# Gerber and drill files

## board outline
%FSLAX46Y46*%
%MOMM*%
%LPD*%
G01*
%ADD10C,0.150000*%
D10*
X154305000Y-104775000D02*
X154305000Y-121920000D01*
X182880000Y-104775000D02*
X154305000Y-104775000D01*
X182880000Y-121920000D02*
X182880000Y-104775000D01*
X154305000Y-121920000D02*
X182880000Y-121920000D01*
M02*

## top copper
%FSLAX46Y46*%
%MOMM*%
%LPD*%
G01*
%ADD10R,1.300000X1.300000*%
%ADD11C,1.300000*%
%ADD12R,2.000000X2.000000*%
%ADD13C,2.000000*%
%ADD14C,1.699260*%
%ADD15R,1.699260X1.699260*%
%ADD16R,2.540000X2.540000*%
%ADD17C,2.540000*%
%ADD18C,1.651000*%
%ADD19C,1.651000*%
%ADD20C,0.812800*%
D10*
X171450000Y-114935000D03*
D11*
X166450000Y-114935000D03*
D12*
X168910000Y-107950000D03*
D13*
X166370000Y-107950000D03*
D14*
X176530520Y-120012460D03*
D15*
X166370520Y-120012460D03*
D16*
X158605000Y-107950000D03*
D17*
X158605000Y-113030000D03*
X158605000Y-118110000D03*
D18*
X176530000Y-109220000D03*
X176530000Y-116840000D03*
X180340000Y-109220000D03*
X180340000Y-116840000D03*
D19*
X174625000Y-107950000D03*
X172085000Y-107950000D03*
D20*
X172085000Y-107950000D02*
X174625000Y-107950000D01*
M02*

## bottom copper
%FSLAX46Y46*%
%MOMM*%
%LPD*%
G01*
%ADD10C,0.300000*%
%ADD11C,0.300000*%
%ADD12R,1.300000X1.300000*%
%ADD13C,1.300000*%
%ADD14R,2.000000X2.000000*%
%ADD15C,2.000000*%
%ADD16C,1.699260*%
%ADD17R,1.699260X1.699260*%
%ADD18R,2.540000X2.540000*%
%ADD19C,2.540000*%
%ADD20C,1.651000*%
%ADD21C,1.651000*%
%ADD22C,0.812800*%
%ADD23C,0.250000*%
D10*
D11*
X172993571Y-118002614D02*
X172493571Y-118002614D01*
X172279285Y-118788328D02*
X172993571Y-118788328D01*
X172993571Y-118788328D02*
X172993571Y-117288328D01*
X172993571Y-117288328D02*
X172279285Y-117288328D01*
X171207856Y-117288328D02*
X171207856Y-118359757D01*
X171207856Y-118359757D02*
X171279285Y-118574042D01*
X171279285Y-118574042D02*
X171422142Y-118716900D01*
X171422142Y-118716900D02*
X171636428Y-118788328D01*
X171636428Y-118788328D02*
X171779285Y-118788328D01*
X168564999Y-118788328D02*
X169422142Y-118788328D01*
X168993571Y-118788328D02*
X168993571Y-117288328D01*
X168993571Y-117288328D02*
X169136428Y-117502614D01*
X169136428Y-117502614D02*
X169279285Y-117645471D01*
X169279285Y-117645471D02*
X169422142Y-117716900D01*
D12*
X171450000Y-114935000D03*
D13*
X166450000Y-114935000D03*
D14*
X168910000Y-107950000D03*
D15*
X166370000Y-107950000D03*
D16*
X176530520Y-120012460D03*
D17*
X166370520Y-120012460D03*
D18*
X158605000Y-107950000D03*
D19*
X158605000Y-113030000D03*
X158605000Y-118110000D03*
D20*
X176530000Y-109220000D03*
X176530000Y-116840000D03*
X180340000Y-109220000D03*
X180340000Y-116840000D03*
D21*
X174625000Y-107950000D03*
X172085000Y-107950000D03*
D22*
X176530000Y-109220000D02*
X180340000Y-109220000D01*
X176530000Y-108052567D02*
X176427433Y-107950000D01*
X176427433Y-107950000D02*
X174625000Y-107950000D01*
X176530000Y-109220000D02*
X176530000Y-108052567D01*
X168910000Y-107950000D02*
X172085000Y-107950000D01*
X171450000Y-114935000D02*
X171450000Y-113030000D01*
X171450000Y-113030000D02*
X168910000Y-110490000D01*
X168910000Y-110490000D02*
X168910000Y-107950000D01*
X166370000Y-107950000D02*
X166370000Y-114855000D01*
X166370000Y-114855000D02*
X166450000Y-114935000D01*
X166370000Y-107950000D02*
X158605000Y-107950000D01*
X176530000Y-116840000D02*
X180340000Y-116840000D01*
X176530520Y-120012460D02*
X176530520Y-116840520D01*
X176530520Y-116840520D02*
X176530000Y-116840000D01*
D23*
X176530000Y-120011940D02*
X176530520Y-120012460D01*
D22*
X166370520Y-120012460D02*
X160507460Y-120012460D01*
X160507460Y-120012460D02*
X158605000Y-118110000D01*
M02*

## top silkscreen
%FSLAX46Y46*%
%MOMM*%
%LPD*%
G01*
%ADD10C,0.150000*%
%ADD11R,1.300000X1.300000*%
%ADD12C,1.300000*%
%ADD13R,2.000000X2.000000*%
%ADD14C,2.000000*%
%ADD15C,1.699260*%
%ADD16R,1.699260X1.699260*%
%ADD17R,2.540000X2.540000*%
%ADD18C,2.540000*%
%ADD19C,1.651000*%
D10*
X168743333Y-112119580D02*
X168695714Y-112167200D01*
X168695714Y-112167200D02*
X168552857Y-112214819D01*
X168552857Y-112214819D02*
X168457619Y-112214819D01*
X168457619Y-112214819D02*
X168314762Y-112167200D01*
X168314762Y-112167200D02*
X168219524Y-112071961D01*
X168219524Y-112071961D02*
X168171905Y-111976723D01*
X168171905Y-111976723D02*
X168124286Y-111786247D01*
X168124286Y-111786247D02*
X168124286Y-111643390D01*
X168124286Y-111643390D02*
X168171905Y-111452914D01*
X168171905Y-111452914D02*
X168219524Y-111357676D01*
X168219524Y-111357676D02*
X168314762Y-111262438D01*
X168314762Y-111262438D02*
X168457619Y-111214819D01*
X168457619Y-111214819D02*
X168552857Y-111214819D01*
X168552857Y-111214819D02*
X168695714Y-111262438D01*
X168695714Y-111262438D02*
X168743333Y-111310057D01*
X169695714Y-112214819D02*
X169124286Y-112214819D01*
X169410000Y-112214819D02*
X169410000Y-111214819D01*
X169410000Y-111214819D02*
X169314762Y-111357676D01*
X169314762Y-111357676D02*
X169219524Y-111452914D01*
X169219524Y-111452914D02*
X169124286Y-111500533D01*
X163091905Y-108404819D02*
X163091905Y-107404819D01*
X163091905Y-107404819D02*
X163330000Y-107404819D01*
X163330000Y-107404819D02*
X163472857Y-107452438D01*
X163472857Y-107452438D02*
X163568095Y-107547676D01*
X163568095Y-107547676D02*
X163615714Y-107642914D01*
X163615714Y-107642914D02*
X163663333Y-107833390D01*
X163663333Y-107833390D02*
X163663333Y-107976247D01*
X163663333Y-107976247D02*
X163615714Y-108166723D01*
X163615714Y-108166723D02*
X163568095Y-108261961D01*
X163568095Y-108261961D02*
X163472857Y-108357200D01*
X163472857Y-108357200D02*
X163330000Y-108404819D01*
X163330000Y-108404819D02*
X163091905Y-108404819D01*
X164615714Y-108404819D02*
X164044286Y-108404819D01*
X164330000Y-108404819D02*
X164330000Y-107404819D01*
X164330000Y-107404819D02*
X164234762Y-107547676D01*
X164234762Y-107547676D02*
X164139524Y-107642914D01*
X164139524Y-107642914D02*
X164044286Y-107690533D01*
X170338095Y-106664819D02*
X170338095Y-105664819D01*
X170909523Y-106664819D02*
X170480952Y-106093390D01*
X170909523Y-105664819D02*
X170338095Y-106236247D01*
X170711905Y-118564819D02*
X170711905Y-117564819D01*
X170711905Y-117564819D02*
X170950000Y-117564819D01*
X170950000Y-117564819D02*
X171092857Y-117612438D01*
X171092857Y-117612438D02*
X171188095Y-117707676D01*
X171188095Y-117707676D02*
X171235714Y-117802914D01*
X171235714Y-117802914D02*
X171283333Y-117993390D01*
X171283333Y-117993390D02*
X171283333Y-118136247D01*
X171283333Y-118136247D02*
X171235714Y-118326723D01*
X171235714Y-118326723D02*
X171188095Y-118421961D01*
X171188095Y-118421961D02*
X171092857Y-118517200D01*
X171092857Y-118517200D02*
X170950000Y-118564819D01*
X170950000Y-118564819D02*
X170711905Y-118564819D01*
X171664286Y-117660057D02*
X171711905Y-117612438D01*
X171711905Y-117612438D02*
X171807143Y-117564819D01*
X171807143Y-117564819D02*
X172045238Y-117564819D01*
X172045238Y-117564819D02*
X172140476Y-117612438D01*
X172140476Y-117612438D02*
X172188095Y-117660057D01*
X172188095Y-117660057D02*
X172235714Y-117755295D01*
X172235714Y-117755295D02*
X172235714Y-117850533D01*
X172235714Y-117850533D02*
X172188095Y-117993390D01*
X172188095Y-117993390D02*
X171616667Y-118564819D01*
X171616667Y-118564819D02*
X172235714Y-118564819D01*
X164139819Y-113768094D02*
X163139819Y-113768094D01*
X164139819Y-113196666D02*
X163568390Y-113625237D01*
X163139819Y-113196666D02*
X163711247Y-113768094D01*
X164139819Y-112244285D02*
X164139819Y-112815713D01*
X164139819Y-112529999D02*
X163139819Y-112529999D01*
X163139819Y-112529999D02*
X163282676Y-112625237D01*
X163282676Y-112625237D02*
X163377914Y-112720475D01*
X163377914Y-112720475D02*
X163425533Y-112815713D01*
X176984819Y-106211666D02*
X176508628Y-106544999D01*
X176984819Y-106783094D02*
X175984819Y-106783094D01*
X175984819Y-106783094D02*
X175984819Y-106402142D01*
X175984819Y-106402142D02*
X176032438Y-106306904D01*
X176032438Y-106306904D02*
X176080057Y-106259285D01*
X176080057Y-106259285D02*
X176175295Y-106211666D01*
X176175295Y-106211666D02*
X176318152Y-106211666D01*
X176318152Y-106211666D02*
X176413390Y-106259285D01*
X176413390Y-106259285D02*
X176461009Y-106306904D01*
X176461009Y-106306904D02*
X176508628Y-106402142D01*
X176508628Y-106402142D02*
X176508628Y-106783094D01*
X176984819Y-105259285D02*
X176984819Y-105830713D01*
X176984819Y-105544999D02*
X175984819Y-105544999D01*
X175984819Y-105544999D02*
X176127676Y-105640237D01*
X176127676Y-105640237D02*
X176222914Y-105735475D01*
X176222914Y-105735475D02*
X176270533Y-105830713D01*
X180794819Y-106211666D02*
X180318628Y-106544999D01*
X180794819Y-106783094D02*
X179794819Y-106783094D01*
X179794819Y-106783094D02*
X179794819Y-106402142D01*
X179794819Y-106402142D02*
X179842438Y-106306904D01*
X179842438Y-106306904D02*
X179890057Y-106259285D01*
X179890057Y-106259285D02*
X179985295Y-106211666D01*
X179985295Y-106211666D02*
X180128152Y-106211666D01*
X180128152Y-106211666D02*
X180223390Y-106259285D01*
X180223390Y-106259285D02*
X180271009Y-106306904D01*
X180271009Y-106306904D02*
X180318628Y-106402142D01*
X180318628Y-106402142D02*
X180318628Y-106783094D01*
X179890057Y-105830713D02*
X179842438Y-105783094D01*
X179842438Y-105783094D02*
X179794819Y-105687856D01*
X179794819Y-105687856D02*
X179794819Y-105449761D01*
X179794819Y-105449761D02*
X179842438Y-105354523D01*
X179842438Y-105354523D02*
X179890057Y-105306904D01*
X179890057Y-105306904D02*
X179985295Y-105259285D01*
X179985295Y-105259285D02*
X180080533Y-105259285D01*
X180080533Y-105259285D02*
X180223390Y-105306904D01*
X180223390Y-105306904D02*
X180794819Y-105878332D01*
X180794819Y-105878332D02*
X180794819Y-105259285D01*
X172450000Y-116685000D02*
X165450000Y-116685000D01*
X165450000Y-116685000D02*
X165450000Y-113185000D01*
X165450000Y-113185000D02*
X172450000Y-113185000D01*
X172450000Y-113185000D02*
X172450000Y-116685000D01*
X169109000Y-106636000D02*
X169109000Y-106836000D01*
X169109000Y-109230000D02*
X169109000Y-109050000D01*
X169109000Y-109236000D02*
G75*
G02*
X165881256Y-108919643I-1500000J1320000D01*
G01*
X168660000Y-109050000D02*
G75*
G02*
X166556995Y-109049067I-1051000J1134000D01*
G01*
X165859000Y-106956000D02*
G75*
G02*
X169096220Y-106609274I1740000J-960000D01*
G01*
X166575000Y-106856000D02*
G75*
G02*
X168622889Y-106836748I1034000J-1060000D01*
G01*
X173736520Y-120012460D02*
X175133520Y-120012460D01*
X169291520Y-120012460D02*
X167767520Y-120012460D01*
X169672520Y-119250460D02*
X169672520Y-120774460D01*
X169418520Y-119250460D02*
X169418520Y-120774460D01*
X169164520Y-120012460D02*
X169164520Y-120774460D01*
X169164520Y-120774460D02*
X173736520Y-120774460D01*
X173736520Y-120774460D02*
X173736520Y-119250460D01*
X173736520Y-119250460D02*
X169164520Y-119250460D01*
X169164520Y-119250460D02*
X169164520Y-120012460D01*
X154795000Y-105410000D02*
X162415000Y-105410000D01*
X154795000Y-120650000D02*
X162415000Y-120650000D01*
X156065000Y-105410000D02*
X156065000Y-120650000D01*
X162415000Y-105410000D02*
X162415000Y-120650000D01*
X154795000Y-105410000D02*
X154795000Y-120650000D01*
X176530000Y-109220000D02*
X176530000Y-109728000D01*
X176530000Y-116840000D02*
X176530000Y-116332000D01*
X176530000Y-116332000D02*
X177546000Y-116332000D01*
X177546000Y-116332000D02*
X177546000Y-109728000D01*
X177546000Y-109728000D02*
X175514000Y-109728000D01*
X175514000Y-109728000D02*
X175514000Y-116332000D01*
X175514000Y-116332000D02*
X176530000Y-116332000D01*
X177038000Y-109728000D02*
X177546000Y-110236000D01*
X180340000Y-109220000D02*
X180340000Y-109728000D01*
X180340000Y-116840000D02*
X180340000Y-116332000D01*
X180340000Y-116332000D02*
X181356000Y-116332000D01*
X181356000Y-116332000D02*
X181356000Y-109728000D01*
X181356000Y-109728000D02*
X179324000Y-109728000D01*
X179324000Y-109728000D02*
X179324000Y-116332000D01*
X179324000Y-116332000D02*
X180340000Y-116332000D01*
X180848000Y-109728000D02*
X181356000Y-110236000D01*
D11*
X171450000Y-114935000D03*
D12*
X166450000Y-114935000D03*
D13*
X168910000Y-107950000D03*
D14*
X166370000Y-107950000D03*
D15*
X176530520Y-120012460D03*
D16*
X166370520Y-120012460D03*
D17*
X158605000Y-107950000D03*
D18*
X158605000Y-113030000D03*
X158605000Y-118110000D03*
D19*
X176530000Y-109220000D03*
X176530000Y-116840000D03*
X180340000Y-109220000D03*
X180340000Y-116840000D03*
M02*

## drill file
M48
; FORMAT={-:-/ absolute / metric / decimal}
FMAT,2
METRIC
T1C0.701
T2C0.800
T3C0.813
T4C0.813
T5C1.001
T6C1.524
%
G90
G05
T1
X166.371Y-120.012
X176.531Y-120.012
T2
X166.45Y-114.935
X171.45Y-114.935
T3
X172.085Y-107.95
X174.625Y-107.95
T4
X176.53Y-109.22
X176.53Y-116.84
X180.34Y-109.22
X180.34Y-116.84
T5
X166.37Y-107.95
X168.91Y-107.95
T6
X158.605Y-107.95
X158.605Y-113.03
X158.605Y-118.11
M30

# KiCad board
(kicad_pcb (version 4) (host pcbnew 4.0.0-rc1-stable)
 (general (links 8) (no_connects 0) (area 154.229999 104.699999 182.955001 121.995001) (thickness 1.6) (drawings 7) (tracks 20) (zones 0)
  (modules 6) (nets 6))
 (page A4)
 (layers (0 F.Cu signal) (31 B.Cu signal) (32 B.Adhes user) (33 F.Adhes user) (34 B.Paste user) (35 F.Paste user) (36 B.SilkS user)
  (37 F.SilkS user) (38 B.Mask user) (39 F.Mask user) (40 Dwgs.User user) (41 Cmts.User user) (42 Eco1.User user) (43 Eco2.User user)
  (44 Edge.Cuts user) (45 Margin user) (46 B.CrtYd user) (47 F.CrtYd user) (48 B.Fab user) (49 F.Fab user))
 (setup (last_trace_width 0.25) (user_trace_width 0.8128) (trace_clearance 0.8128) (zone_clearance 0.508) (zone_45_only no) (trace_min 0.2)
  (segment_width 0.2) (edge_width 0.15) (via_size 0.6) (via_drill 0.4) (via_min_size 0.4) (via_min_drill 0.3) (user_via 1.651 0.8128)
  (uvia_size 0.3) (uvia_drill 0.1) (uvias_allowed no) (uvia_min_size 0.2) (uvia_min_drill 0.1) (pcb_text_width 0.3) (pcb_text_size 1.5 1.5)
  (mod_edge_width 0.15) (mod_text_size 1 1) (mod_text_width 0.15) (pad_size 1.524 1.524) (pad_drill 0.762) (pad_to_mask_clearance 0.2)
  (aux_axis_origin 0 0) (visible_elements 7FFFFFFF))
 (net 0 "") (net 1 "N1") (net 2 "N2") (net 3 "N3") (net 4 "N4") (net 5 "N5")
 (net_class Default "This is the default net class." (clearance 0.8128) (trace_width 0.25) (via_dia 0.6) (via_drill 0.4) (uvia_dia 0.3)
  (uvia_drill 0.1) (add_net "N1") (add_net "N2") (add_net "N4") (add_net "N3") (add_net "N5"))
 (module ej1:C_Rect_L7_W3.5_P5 (layer F.Cu) (at 171.45 114.935 180)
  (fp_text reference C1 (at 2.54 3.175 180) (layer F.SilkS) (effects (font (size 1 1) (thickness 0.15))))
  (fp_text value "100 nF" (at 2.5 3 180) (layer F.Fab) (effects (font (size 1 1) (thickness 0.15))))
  (fp_line (start -1 -1.75) (end 6 -1.75) (layer F.SilkS) (width 0.15))
  (fp_line (start 6 -1.75) (end 6 1.75) (layer F.SilkS) (width 0.15))
  (fp_line (start 6 1.75) (end -1 1.75) (layer F.SilkS) (width 0.15))
  (fp_line (start -1 1.75) (end -1 -1.75) (layer F.SilkS) (width 0.15))
  (pad 1 thru_hole rect (at 0 0 180) (size 1.3 1.3) (drill 0.8) (layers *.Cu *.Mask F.SilkS) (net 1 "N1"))
  (pad 2 thru_hole circle (at 5 0 180) (size 1.3 1.3) (drill 0.8) (layers *.Cu *.Mask F.SilkS) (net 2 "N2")))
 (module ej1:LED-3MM (layer F.Cu) (at 168.91 107.95 180)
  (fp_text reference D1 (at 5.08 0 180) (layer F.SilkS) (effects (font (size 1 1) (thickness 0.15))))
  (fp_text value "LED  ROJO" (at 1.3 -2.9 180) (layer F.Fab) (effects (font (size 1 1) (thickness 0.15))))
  (fp_line (start -0.199 1.314) (end -0.199 1.114) (layer F.SilkS) (width 0.15))
  (fp_line (start -0.199 -1.28) (end -0.199 -1.1) (layer F.SilkS) (width 0.15))
  (fp_arc (start 1.301 0.034) (end -0.199 -1.286) (angle 108.5) (layer F.SilkS) (width 0.15))
  (fp_arc (start 1.301 0.034) (end 0.25 -1.1) (angle 85.7) (layer F.SilkS) (width 0.15))
  (fp_arc (start 1.311 0.034) (end 3.051 0.994) (angle 110) (layer F.SilkS) (width 0.15))
  (fp_arc (start 1.301 0.034) (end 2.335 1.094) (angle 87.5) (layer F.SilkS) (width 0.15))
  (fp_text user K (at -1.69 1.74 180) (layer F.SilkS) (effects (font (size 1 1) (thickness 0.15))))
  (pad 1 thru_hole rect (at 0 0 270) (size 2 2) (drill 1.00076) (layers *.Cu *.Mask F.SilkS) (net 1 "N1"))
  (pad 2 thru_hole circle (at 2.54 0 180) (size 2 2) (drill 1.00076) (layers *.Cu *.Mask F.SilkS) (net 2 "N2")))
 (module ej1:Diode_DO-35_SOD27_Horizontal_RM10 (layer F.Cu) (at 166.37 120.015)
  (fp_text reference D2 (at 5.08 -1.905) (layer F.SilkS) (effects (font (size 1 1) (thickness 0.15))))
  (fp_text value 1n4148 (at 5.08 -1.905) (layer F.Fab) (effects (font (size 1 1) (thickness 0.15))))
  (fp_line (start 7.36652 -0.00254) (end 8.76352 -0.00254) (layer F.SilkS) (width 0.15))
  (fp_line (start 2.92152 -0.00254) (end 1.39752 -0.00254) (layer F.SilkS) (width 0.15))
  (fp_line (start 3.30252 -0.76454) (end 3.30252 0.75946) (layer F.SilkS) (width 0.15))
  (fp_line (start 3.04852 -0.76454) (end 3.04852 0.75946) (layer F.SilkS) (width 0.15))
  (fp_line (start 2.79452 -0.00254) (end 2.79452 0.75946) (layer F.SilkS) (width 0.15))
  (fp_line (start 2.79452 0.75946) (end 7.36652 0.75946) (layer F.SilkS) (width 0.15))
  (fp_line (start 7.36652 0.75946) (end 7.36652 -0.76454) (layer F.SilkS) (width 0.15))
  (fp_line (start 7.36652 -0.76454) (end 2.79452 -0.76454) (layer F.SilkS) (width 0.15))
  (fp_line (start 2.79452 -0.76454) (end 2.79452 -0.00254) (layer F.SilkS) (width 0.15))
  (pad 2 thru_hole circle (at 10.16052 -0.00254 180) (size 1.69926 1.69926) (drill 0.70104) (layers *.Cu *.Mask F.SilkS) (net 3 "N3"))
  (pad 1 thru_hole rect (at 0.00052 -0.00254 180) (size 1.69926 1.69926) (drill 0.70104) (layers *.Cu *.Mask F.SilkS) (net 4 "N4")))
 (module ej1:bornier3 (layer F.Cu) (at 158.605 113.03 270)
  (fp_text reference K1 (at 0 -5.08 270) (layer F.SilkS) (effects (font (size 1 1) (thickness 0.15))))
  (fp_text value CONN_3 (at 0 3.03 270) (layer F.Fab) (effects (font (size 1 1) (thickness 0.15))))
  (fp_line (start -7.62 3.81) (end -7.62 -3.81) (layer F.SilkS) (width 0.15))
  (fp_line (start 7.62 3.81) (end 7.62 -3.81) (layer F.SilkS) (width 0.15))
  (fp_line (start -7.62 2.54) (end 7.62 2.54) (layer F.SilkS) (width 0.15))
  (fp_line (start -7.62 -3.81) (end 7.62 -3.81) (layer F.SilkS) (width 0.15))
  (fp_line (start -7.62 3.81) (end 7.62 3.81) (layer F.SilkS) (width 0.15))
  (pad 1 thru_hole rect (at -5.08 0 270) (size 2.54 2.54) (drill 1.524) (layers *.Cu *.Mask F.SilkS) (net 2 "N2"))
  (pad 2 thru_hole circle (at 0 0 270) (size 2.54 2.54) (drill 1.524) (layers *.Cu *.Mask F.SilkS) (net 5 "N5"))
  (pad 3 thru_hole circle (at 5.08 0 270) (size 2.54 2.54) (drill 1.524) (layers *.Cu *.Mask F.SilkS) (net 4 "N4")))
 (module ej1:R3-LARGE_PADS (layer F.Cu) (at 176.53 113.03 270)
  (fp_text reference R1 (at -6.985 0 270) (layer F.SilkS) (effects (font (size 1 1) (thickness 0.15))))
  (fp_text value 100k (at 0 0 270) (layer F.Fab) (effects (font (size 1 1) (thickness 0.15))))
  (fp_line (start -3.81 0) (end -3.302 0) (layer F.SilkS) (width 0.15))
  (fp_line (start 3.81 0) (end 3.302 0) (layer F.SilkS) (width 0.15))
  (fp_line (start 3.302 0) (end 3.302 -1.016) (layer F.SilkS) (width 0.15))
  (fp_line (start 3.302 -1.016) (end -3.302 -1.016) (layer F.SilkS) (width 0.15))
  (fp_line (start -3.302 -1.016) (end -3.302 1.016) (layer F.SilkS) (width 0.15))
  (fp_line (start -3.302 1.016) (end 3.302 1.016) (layer F.SilkS) (width 0.15))
  (fp_line (start 3.302 1.016) (end 3.302 0) (layer F.SilkS) (width 0.15))
  (fp_line (start -3.302 -0.508) (end -2.794 -1.016) (layer F.SilkS) (width 0.15))
  (pad 1 thru_hole circle (at -3.81 0 270) (size 1.651 1.651) (drill 0.8128) (layers *.Cu *.Mask F.SilkS) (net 1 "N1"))
  (pad 2 thru_hole circle (at 3.81 0 270) (size 1.651 1.651) (drill 0.8128) (layers *.Cu *.Mask F.SilkS) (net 3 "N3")))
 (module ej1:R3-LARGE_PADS (layer F.Cu) (at 180.34 113.03 270)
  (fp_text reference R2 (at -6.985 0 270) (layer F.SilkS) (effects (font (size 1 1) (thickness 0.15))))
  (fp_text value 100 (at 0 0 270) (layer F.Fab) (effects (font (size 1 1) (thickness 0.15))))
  (fp_line (start -3.81 0) (end -3.302 0) (layer F.SilkS) (width 0.15))
  (fp_line (start 3.81 0) (end 3.302 0) (layer F.SilkS) (width 0.15))
  (fp_line (start 3.302 0) (end 3.302 -1.016) (layer F.SilkS) (width 0.15))
  (fp_line (start 3.302 -1.016) (end -3.302 -1.016) (layer F.SilkS) (width 0.15))
  (fp_line (start -3.302 -1.016) (end -3.302 1.016) (layer F.SilkS) (width 0.15))
  (fp_line (start -3.302 1.016) (end 3.302 1.016) (layer F.SilkS) (width 0.15))
  (fp_line (start 3.302 1.016) (end 3.302 0) (layer F.SilkS) (width 0.15))
  (fp_line (start -3.302 -0.508) (end -2.794 -1.016) (layer F.SilkS) (width 0.15))
  (pad 1 thru_hole circle (at -3.81 0 270) (size 1.651 1.651) (drill 0.8128) (layers *.Cu *.Mask F.SilkS) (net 1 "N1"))
  (pad 2 thru_hole circle (at 3.81 0 270) (size 1.651 1.651) (drill 0.8128) (layers *.Cu *.Mask F.SilkS) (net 3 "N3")))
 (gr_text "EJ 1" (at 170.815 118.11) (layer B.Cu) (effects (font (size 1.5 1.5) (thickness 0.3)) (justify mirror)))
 (gr_line (start 154.305 104.775) (end 154.305 121.92) (layer Edge.Cuts) (width 0.15))
 (gr_line (start 182.88 104.775) (end 154.305 104.775) (layer Edge.Cuts) (width 0.15))
 (gr_line (start 182.88 121.92) (end 182.88 104.775) (layer Edge.Cuts) (width 0.15))
 (gr_line (start 154.305 121.92) (end 182.88 121.92) (layer Edge.Cuts) (width 0.15))
 (segment (start 176.53 109.22) (end 180.34 109.22) (width 0.8128) (layer B.Cu) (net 1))
 (segment (start 176.53 108.052567) (end 176.427433 107.95) (width 0.8128) (layer B.Cu) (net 1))
 (segment (start 176.427433 107.95) (end 174.625 107.95) (width 0.8128) (layer B.Cu) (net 1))
 (segment (start 176.53 109.22) (end 176.53 108.052567) (width 0.8128) (layer B.Cu) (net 1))
 (via (at 174.625 107.95) (size 1.651) (drill 0.8128) (layers F.Cu B.Cu) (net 1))
 (segment (start 172.085 107.95) (end 174.625 107.95) (width 0.8128) (layer F.Cu) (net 1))
 (via (at 172.085 107.95) (size 1.651) (drill 0.8128) (layers F.Cu B.Cu) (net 1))
 (segment (start 168.91 107.95) (end 172.085 107.95) (width 0.8128) (layer B.Cu) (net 1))
 (segment (start 171.45 114.935) (end 171.45 113.03) (width 0.8128) (layer B.Cu) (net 1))
 (segment (start 171.45 113.03) (end 168.91 110.49) (width 0.8128) (layer B.Cu) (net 1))
 (segment (start 168.91 110.49) (end 168.91 107.95) (width 0.8128) (layer B.Cu) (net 1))
 (segment (start 166.37 107.95) (end 166.37 114.855) (width 0.8128) (layer B.Cu) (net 2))
 (segment (start 166.37 114.855) (end 166.45 114.935) (width 0.8128) (layer B.Cu) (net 2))
 (segment (start 166.37 107.95) (end 158.605 107.95) (width 0.8128) (layer B.Cu) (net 2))
 (segment (start 176.53 116.84) (end 180.34 116.84) (width 0.8128) (layer B.Cu) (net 3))
 (segment (start 176.53052 120.01246) (end 176.53052 116.84052) (width 0.8128) (layer B.Cu) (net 3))
 (segment (start 176.53052 116.84052) (end 176.53 116.84) (width 0.8128) (layer B.Cu) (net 3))
 (segment (start 176.53 120.01194) (end 176.53052 120.01246) (width 0.25) (layer B.Cu) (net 3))
 (segment (start 166.37052 120.01246) (end 160.50746 120.01246) (width 0.8128) (layer B.Cu) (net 4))
 (segment (start 160.50746 120.01246) (end 158.605 118.11) (width 0.8128) (layer B.Cu) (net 4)))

